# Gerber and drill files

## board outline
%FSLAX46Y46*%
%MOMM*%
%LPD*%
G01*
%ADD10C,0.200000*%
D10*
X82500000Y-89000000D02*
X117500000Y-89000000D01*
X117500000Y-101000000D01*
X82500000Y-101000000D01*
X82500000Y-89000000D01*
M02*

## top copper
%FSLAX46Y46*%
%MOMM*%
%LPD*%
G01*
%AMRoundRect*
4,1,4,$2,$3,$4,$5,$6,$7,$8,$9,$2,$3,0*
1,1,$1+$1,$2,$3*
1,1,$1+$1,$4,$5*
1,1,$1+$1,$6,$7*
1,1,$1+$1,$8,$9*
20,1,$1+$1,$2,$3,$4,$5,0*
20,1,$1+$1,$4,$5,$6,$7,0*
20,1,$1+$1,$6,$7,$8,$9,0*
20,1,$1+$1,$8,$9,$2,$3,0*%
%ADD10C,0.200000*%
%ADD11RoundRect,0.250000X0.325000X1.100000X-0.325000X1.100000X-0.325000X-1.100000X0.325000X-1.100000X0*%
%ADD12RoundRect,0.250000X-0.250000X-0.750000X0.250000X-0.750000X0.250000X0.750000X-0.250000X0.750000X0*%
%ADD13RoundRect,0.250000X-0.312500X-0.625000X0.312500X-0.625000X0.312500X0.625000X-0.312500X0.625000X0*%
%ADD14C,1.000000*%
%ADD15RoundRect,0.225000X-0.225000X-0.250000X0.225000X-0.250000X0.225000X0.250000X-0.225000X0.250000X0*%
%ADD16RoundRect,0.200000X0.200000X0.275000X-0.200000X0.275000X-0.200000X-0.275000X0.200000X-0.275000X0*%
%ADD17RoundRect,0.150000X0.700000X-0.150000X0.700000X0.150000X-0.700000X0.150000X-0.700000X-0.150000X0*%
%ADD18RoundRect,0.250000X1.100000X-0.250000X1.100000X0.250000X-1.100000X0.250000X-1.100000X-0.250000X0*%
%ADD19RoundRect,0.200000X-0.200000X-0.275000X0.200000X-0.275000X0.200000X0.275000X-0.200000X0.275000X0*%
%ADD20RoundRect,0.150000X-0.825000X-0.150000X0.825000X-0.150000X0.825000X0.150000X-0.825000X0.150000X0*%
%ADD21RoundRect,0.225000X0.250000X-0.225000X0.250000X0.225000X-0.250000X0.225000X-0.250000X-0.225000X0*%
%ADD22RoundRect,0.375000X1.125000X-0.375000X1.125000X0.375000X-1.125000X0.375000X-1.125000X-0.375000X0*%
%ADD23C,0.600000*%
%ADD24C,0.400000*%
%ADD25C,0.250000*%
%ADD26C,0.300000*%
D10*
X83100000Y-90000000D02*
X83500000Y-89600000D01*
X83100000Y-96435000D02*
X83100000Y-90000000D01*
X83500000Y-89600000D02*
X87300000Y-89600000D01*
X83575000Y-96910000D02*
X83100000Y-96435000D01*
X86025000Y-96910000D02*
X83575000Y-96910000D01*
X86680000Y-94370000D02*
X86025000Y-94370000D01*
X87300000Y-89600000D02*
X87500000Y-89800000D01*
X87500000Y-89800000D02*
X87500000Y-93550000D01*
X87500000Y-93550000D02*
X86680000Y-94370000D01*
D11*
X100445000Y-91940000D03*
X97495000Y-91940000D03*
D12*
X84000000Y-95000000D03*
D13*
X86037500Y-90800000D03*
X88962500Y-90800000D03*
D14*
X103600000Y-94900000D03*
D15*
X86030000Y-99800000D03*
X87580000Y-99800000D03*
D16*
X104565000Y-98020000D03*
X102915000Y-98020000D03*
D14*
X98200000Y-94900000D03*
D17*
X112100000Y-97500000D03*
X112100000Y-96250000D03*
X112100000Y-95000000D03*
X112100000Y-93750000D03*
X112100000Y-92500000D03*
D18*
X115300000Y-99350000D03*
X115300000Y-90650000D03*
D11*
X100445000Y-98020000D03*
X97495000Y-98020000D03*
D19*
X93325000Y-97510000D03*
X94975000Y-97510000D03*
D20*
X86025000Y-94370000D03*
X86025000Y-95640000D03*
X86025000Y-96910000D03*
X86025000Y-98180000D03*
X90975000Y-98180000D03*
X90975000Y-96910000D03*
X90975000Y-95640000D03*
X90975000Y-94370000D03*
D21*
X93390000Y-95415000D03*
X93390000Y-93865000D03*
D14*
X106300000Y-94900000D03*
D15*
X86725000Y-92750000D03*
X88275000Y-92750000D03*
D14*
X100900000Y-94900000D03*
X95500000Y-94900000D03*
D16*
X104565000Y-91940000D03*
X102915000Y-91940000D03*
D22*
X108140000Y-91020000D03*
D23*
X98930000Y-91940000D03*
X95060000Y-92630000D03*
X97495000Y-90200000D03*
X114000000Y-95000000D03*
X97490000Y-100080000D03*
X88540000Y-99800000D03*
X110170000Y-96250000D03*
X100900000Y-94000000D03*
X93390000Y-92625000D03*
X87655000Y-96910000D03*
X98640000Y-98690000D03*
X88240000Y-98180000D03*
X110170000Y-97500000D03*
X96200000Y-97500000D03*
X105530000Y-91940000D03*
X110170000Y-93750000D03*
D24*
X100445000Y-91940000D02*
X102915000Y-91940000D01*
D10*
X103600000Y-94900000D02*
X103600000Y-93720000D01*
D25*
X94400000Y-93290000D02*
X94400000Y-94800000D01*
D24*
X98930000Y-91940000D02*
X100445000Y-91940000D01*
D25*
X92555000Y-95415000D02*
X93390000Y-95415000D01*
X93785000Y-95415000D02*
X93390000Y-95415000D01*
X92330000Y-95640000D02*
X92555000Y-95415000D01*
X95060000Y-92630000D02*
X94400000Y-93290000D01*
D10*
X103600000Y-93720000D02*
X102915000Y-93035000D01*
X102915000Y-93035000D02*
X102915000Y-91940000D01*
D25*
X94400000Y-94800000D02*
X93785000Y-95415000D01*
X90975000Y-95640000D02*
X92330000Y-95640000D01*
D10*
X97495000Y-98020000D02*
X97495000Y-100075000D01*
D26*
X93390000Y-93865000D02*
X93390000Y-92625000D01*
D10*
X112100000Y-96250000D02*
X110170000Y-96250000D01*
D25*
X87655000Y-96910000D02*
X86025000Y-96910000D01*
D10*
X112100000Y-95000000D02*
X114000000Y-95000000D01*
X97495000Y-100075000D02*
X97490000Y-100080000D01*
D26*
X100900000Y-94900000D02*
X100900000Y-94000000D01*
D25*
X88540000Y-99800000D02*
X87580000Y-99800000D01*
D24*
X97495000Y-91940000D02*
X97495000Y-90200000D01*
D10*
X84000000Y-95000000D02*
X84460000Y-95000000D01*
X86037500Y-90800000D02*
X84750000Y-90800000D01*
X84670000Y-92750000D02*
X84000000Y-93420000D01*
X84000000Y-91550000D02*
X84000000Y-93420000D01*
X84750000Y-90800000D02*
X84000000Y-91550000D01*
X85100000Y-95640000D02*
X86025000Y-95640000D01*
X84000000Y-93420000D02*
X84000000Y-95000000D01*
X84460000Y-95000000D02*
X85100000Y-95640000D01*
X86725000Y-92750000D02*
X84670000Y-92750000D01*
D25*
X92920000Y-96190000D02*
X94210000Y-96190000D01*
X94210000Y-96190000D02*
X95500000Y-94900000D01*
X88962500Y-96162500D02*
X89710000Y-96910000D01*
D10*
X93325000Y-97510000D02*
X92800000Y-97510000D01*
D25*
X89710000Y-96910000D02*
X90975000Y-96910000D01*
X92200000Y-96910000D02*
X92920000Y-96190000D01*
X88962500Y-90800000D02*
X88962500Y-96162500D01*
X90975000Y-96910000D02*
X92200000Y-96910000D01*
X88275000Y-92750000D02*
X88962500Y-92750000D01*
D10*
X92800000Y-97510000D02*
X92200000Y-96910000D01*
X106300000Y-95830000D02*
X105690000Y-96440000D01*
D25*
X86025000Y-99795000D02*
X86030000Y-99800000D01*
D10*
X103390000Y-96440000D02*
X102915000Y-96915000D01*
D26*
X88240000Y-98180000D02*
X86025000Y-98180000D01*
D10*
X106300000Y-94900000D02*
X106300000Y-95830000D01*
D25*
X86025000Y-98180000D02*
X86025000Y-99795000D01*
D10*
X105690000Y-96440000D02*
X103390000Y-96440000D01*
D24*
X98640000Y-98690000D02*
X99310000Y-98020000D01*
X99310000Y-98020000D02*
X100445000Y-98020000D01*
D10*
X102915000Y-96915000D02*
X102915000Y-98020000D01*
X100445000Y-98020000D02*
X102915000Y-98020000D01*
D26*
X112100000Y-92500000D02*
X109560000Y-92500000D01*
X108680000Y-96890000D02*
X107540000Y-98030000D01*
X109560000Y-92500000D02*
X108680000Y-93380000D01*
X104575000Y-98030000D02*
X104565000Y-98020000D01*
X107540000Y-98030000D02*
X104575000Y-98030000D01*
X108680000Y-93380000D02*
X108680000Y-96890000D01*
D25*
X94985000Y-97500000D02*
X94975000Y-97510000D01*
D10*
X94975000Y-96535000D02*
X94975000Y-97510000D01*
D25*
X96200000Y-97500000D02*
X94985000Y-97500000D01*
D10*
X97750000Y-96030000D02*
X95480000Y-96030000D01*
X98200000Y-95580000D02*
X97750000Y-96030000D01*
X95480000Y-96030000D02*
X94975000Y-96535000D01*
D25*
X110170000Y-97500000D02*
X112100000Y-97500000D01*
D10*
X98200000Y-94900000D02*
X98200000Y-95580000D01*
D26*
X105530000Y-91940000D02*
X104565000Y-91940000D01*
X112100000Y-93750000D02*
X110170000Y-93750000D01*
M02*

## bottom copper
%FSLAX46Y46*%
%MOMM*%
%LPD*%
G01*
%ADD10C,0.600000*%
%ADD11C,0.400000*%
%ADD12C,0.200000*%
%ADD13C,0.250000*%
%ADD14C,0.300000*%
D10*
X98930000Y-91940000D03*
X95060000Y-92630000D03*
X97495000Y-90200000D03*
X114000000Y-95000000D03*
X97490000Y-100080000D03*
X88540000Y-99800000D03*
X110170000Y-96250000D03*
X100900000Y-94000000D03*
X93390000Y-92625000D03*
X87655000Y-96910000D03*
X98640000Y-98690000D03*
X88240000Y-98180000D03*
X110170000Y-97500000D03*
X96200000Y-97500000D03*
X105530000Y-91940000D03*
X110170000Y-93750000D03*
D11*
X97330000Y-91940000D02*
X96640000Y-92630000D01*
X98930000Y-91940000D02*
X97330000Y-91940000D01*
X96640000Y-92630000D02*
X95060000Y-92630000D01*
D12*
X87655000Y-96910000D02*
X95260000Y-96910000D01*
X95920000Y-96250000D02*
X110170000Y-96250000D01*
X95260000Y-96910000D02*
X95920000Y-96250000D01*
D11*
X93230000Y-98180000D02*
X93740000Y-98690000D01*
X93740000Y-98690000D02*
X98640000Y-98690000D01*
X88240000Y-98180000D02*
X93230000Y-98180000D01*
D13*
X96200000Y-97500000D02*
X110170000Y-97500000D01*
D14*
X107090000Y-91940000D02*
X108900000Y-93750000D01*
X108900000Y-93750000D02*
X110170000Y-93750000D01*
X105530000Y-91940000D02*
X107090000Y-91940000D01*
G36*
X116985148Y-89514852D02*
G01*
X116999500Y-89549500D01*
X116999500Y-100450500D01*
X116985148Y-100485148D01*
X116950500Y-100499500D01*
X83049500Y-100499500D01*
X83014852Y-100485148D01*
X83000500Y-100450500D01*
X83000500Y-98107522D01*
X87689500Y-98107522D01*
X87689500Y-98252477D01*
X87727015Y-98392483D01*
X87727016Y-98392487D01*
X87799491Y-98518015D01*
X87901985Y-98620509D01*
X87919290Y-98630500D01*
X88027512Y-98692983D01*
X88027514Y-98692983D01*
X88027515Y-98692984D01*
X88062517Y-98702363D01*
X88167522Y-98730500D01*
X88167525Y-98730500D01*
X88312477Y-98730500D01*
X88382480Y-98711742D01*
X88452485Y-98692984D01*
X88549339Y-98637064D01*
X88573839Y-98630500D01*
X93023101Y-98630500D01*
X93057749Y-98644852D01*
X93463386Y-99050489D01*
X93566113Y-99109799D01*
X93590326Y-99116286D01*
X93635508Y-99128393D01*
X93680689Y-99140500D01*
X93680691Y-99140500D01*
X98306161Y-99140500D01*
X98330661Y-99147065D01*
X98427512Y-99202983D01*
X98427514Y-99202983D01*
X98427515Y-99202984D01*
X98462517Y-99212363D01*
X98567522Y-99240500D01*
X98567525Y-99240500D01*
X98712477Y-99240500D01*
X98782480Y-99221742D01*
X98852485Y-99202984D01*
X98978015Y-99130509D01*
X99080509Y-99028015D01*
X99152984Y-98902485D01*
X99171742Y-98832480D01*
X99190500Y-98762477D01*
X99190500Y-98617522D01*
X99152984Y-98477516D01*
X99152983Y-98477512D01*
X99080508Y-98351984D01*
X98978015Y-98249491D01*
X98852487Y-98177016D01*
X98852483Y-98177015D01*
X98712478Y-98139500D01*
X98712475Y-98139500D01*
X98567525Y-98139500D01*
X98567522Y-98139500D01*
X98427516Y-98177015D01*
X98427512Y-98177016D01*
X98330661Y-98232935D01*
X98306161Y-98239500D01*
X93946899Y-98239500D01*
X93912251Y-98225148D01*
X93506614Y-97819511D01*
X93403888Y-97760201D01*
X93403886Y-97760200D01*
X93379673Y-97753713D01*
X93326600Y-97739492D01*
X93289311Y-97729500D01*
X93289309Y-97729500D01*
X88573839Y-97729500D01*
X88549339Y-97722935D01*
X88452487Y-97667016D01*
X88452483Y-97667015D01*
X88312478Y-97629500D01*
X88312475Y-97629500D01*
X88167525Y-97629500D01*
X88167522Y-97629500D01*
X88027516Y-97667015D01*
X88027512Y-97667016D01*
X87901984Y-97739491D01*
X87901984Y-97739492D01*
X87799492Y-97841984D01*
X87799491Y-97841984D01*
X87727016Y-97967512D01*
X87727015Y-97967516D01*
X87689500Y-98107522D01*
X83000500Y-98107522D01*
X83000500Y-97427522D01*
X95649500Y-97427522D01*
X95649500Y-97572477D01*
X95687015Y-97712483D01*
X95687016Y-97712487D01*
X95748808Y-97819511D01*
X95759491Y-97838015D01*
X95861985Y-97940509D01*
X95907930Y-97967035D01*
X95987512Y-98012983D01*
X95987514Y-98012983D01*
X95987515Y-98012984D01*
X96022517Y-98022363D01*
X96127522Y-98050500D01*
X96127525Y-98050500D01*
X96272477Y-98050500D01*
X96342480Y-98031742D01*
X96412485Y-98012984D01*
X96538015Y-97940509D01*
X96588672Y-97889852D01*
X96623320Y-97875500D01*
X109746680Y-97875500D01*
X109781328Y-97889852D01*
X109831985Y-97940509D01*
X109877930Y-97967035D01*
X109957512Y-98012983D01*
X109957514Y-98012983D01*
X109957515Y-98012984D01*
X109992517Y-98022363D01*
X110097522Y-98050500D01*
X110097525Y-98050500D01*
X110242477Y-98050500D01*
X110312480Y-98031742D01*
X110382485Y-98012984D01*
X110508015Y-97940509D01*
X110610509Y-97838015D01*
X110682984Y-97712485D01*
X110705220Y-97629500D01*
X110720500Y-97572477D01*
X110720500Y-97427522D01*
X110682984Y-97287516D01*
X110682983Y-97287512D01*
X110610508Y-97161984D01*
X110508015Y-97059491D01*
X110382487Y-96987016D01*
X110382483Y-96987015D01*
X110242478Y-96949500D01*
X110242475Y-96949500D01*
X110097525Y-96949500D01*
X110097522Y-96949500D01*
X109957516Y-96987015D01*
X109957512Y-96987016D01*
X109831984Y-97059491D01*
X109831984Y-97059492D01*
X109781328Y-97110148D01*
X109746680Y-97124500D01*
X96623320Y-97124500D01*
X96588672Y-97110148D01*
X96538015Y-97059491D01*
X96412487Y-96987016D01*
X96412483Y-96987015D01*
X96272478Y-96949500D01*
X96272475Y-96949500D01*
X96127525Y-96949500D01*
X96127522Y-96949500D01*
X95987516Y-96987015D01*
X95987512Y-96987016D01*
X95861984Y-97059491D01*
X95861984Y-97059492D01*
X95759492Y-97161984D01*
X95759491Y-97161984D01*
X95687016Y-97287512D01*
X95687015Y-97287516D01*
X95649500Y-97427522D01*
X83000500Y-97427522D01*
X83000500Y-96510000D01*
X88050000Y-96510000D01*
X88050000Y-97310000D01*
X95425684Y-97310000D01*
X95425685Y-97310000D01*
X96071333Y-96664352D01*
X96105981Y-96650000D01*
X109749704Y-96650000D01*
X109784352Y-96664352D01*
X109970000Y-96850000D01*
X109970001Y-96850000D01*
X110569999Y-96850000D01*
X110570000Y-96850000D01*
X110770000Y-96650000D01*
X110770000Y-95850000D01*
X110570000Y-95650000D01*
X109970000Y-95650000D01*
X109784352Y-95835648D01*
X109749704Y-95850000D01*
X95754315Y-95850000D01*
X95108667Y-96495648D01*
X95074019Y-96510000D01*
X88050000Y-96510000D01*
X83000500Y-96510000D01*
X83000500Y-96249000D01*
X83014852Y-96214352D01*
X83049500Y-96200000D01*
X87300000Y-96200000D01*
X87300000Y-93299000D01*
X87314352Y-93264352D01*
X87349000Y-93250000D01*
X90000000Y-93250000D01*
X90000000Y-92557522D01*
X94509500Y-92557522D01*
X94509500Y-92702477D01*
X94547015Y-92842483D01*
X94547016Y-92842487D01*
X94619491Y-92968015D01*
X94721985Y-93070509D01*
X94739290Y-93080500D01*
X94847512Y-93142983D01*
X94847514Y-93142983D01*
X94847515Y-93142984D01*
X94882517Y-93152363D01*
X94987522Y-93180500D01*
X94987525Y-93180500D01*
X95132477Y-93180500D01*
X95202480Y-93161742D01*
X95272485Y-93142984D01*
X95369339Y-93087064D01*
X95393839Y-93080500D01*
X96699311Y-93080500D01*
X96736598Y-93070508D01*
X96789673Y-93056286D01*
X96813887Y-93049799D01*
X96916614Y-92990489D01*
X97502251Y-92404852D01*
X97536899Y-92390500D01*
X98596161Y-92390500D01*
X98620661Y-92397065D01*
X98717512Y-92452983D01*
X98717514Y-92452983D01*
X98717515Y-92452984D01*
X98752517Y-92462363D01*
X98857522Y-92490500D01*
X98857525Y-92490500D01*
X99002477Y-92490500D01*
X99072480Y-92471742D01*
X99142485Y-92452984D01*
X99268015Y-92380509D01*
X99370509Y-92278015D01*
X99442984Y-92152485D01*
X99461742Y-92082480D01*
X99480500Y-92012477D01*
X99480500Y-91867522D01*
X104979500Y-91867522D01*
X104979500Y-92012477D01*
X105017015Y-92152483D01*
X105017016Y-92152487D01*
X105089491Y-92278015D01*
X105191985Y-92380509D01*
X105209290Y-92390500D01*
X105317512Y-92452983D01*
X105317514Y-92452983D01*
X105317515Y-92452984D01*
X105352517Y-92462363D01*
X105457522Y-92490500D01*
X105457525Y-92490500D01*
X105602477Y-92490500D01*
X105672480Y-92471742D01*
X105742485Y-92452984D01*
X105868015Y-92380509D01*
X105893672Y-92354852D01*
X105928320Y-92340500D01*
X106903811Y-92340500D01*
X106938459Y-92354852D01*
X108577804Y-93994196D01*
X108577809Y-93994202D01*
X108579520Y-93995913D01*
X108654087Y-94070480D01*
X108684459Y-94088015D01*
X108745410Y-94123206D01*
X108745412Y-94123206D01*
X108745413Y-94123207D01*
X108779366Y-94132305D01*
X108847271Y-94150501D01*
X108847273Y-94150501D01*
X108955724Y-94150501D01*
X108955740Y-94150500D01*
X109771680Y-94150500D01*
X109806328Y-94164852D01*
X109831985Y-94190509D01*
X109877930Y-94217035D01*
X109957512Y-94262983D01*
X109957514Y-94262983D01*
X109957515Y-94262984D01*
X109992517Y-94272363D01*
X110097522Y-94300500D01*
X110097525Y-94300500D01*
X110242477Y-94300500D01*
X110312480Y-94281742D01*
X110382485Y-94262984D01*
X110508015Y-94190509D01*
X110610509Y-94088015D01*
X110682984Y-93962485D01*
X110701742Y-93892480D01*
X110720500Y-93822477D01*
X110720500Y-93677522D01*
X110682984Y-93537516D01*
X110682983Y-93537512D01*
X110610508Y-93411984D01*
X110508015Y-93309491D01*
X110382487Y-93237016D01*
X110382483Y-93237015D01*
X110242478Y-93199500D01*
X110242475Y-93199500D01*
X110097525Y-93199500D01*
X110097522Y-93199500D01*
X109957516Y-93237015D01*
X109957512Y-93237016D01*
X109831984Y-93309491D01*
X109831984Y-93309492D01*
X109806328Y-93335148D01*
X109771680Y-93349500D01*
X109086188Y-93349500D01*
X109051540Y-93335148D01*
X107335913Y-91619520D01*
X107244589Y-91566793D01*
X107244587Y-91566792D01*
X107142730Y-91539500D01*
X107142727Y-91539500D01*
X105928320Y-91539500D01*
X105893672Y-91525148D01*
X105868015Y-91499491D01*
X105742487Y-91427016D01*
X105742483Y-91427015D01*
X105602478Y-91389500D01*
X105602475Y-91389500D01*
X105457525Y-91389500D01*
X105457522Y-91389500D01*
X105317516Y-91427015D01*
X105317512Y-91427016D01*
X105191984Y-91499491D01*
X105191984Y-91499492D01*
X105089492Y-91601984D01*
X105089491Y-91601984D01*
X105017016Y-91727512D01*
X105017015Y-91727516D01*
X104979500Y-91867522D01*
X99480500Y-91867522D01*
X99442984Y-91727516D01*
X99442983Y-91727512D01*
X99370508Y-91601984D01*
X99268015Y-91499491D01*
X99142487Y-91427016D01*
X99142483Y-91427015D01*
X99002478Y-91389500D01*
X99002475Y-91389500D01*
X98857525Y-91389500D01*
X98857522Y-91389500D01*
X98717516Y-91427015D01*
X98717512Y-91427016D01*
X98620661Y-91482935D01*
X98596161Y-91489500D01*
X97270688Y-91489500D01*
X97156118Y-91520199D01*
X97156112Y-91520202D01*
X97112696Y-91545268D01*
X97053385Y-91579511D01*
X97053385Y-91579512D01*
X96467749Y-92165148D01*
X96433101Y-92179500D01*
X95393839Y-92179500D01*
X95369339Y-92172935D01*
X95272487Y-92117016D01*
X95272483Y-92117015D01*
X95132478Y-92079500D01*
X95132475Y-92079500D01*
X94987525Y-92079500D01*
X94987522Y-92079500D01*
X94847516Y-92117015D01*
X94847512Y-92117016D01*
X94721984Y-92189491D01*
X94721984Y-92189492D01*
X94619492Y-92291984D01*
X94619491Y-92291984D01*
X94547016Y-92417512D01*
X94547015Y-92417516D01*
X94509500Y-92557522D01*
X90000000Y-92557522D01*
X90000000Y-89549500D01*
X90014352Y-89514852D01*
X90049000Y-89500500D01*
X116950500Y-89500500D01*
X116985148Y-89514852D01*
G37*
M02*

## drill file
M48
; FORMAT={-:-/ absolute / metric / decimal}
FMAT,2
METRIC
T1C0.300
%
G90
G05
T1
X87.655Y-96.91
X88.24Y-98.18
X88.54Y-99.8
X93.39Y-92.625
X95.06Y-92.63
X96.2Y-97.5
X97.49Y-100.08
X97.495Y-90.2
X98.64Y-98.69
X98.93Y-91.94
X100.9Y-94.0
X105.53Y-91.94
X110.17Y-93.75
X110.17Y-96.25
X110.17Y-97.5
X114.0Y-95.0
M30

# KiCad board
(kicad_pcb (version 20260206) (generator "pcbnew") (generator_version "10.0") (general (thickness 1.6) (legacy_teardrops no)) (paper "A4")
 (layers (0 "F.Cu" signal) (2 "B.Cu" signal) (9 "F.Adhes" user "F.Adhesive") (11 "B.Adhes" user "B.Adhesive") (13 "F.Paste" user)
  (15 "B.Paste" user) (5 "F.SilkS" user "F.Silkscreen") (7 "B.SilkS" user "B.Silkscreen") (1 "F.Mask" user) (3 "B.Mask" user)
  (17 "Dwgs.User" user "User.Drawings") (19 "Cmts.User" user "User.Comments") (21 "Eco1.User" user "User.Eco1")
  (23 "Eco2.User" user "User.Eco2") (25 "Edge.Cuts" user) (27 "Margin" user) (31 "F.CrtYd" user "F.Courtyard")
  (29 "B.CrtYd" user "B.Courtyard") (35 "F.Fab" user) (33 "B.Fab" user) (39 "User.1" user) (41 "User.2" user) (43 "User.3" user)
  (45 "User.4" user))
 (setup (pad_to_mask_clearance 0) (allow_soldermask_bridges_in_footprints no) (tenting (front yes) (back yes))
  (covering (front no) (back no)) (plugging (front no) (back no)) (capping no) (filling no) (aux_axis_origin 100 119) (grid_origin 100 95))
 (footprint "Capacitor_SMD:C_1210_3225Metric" (layer "F.Cu") (at 98.97 91.94 180)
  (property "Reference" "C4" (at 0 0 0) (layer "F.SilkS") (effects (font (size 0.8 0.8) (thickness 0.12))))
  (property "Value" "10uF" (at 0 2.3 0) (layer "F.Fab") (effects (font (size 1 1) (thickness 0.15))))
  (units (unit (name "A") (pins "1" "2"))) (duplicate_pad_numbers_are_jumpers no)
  (pad "1" smd roundrect (at -1.475 0 180) (size 1.15 2.7) (layers "F.Cu" "F.Mask" "F.Paste") (roundrect_rratio 0.217391) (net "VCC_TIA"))
  (pad "2" smd roundrect (at 1.475 0 180) (size 1.15 2.7) (layers "F.Cu" "F.Mask" "F.Paste") (roundrect_rratio 0.217391) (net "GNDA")))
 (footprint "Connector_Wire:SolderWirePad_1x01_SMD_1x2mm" (layer "F.Cu") (at 84 95)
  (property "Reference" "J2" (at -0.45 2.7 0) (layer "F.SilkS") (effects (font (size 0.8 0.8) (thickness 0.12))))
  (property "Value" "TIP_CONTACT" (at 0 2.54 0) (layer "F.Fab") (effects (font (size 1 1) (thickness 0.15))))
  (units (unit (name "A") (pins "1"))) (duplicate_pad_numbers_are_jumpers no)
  (pad "1" smd roundrect (at 0 0) (size 1 2) (layers "F.Cu" "F.Mask") (roundrect_rratio 0.25) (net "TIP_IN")))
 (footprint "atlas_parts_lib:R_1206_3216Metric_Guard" (layer "F.Cu") (at 87.5 90.8)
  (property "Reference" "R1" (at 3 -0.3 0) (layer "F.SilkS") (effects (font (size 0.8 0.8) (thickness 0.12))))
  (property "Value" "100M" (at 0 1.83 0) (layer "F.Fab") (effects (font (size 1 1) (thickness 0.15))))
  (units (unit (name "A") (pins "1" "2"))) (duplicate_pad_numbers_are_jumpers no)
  (pad "1" smd roundrect (at -1.4625 0) (size 1.125 1.75) (layers "F.Cu" "F.Mask" "F.Paste") (roundrect_rratio 0.222222) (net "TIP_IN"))
  (pad "2" smd roundrect (at 1.4625 0) (size 1.125 1.75) (layers "F.Cu" "F.Mask" "F.Paste") (roundrect_rratio 0.222222) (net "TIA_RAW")))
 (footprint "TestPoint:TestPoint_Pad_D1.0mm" (layer "F.Cu") (at 103.6 94.9)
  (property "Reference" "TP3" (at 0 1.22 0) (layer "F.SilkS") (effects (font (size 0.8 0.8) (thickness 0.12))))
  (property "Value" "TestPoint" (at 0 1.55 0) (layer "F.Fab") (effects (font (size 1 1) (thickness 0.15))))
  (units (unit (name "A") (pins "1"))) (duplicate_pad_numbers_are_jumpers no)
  (pad "1" smd circle (at 0 0) (size 1 1) (layers "F.Cu" "F.Mask") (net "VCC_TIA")))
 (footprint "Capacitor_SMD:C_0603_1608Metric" (layer "F.Cu") (at 86.805 99.8)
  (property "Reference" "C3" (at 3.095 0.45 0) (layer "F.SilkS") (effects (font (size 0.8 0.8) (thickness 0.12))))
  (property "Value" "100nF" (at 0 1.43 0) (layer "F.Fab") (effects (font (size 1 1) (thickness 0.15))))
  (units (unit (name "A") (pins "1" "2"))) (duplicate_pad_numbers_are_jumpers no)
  (pad "1" smd roundrect (at -0.775 0) (size 0.9 0.95) (layers "F.Cu" "F.Mask" "F.Paste") (roundrect_rratio 0.25) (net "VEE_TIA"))
  (pad "2" smd roundrect (at 0.775 0) (size 0.9 0.95) (layers "F.Cu" "F.Mask" "F.Paste") (roundrect_rratio 0.25) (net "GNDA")))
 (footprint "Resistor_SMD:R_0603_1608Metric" (layer "F.Cu") (at 103.74 98.02 180)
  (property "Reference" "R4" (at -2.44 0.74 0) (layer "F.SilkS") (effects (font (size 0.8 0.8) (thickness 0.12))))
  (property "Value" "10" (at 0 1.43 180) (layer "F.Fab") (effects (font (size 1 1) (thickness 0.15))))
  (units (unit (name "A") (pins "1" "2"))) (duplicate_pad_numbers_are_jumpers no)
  (pad "1" smd roundrect (at -0.825 0 180) (size 0.8 0.95) (layers "F.Cu" "F.Mask" "F.Paste") (roundrect_rratio 0.25) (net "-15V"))
  (pad "2" smd roundrect (at 0.825 0 180) (size 0.8 0.95) (layers "F.Cu" "F.Mask" "F.Paste") (roundrect_rratio 0.25) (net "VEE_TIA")))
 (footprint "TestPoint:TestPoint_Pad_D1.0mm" (layer "F.Cu") (at 98.2 94.9)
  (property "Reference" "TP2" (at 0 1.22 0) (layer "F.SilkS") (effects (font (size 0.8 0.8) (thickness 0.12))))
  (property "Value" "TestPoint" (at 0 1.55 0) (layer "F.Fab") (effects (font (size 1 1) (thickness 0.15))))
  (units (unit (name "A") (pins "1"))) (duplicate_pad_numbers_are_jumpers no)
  (pad "1" smd circle (at 0 0) (size 1 1) (layers "F.Cu" "F.Mask") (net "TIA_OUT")))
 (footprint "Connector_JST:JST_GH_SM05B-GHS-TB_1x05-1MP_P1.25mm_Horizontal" (layer "F.Cu") (at 113.95 95 90)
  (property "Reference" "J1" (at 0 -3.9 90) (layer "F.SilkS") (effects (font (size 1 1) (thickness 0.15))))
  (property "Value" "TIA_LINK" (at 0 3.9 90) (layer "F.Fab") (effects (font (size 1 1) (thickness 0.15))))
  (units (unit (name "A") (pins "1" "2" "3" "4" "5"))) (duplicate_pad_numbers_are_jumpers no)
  (pad "1" smd roundrect (at -2.5 -1.85 90) (size 0.6 1.7) (layers "F.Cu" "F.Mask" "F.Paste") (roundrect_rratio 0.25) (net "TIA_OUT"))
  (pad "2" smd roundrect (at -1.25 -1.85 90) (size 0.6 1.7) (layers "F.Cu" "F.Mask" "F.Paste") (roundrect_rratio 0.25) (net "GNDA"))
  (pad "3" smd roundrect (at 0 -1.85 90) (size 0.6 1.7) (layers "F.Cu" "F.Mask" "F.Paste") (roundrect_rratio 0.25) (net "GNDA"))
  (pad "4" smd roundrect (at 1.25 -1.85 90) (size 0.6 1.7) (layers "F.Cu" "F.Mask" "F.Paste") (roundrect_rratio 0.25) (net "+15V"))
  (pad "5" smd roundrect (at 2.5 -1.85 90) (size 0.6 1.7) (layers "F.Cu" "F.Mask" "F.Paste") (roundrect_rratio 0.25) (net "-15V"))
  (pad "MP" smd roundrect (at -4.35 1.35 90) (size 1 2.7) (layers "F.Cu" "F.Mask" "F.Paste") (roundrect_rratio 0.25))
  (pad "MP" smd roundrect (at 4.35 1.35 90) (size 1 2.7) (layers "F.Cu" "F.Mask" "F.Paste") (roundrect_rratio 0.25)))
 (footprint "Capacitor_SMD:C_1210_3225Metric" (layer "F.Cu") (at 98.97 98.02 180)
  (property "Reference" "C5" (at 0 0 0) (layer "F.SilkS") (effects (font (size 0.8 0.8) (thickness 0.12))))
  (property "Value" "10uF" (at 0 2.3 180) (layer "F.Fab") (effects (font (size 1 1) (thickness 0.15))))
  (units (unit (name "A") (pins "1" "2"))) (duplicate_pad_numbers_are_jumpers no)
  (pad "1" smd roundrect (at -1.475 0 180) (size 1.15 2.7) (layers "F.Cu" "F.Mask" "F.Paste") (roundrect_rratio 0.217391) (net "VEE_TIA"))
  (pad "2" smd roundrect (at 1.475 0 180) (size 1.15 2.7) (layers "F.Cu" "F.Mask" "F.Paste") (roundrect_rratio 0.217391) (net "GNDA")))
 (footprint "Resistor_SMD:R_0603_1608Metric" (layer "F.Cu") (at 94.15 97.51)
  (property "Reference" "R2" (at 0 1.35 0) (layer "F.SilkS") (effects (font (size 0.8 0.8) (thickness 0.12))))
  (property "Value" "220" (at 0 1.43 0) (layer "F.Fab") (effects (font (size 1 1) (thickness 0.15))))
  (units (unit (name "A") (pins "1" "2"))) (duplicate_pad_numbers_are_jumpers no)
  (pad "1" smd roundrect (at -0.825 0) (size 0.8 0.95) (layers "F.Cu" "F.Mask" "F.Paste") (roundrect_rratio 0.25) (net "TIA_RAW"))
  (pad "2" smd roundrect (at 0.825 0) (size 0.8 0.95) (layers "F.Cu" "F.Mask" "F.Paste") (roundrect_rratio 0.25) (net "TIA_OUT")))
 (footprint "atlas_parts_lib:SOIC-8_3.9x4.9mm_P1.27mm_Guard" (layer "F.Cu") (at 88.5 96.275)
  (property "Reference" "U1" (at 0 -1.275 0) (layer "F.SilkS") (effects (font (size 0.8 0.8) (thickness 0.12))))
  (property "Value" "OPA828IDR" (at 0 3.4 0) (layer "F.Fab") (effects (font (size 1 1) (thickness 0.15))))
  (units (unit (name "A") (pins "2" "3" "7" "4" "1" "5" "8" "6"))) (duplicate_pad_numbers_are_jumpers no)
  (pad "1" smd roundrect (at -2.475 -1.905) (size 1.95 0.6) (layers "F.Cu" "F.Mask" "F.Paste") (roundrect_rratio 0.25) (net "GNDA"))
  (pad "2" smd roundrect (at -2.475 -0.635) (size 1.95 0.6) (layers "F.Cu" "F.Mask" "F.Paste") (roundrect_rratio 0.25) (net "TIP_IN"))
  (pad "3" smd roundrect (at -2.475 0.635) (size 1.95 0.6) (layers "F.Cu" "F.Mask" "F.Paste") (roundrect_rratio 0.25) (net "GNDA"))
  (pad "4" smd roundrect (at -2.475 1.905) (size 1.95 0.6) (layers "F.Cu" "F.Mask" "F.Paste") (roundrect_rratio 0.25) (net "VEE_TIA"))
  (pad "5" smd roundrect (at 2.475 1.905) (size 1.95 0.6) (layers "F.Cu" "F.Mask" "F.Paste") (roundrect_rratio 0.25)
   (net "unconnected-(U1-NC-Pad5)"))
  (pad "6" smd roundrect (at 2.475 0.635) (size 1.95 0.6) (layers "F.Cu" "F.Mask" "F.Paste") (roundrect_rratio 0.25) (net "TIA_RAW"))
  (pad "7" smd roundrect (at 2.475 -0.635) (size 1.95 0.6) (layers "F.Cu" "F.Mask" "F.Paste") (roundrect_rratio 0.25) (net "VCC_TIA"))
  (pad "8" smd roundrect (at 2.475 -1.905) (size 1.95 0.6) (layers "F.Cu" "F.Mask" "F.Paste") (roundrect_rratio 0.25)
   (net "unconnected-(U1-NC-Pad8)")))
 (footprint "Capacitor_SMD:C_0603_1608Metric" (layer "F.Cu") (at 93.39 94.64 90)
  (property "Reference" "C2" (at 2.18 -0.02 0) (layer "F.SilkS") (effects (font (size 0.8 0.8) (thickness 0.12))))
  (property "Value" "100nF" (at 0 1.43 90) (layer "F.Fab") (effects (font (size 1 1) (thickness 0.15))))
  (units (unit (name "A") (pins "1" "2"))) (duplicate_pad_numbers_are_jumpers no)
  (pad "1" smd roundrect (at -0.775 0 90) (size 0.9 0.95) (layers "F.Cu" "F.Mask" "F.Paste") (roundrect_rratio 0.25) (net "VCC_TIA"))
  (pad "2" smd roundrect (at 0.775 0 90) (size 0.9 0.95) (layers "F.Cu" "F.Mask" "F.Paste") (roundrect_rratio 0.25) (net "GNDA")))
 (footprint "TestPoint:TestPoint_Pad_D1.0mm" (layer "F.Cu") (at 106.3 94.9)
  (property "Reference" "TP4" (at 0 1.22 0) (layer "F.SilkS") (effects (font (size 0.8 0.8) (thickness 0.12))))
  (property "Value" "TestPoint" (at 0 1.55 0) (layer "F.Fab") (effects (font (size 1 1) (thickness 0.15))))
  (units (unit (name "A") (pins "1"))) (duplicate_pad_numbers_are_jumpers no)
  (pad "1" smd circle (at 0 0) (size 1 1) (layers "F.Cu" "F.Mask") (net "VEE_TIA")))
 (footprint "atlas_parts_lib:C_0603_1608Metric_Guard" (layer "F.Cu") (at 87.5 92.75)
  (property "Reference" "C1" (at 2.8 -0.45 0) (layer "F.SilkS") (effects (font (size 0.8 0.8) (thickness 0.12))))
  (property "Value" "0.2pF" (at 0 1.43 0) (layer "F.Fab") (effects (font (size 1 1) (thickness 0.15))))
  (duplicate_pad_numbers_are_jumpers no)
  (pad "1" smd roundrect (at -0.775 0) (size 0.9 0.95) (layers "F.Cu" "F.Mask" "F.Paste") (roundrect_rratio 0.25) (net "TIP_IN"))
  (pad "2" smd roundrect (at 0.775 0) (size 0.9 0.95) (layers "F.Cu" "F.Mask" "F.Paste") (roundrect_rratio 0.25) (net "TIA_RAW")))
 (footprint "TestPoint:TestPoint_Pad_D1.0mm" (layer "F.Cu") (at 100.9 94.9)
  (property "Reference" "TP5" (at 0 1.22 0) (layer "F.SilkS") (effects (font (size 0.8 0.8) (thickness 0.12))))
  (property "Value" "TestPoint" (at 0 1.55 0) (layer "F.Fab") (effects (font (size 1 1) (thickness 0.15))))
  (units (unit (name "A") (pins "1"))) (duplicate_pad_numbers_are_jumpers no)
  (pad "1" smd circle (at 0 0) (size 1 1) (layers "F.Cu" "F.Mask") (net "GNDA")))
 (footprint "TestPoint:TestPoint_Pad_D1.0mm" (layer "F.Cu") (at 95.5 94.9)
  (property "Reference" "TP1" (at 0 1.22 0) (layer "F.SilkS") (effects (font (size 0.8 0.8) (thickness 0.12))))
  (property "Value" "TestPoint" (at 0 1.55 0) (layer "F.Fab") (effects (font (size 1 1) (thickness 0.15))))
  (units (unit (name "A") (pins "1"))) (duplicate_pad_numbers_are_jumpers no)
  (pad "1" smd circle (at 0 0) (size 1 1) (layers "F.Cu" "F.Mask") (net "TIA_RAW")))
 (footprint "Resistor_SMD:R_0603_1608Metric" (layer "F.Cu") (at 103.74 91.94 180)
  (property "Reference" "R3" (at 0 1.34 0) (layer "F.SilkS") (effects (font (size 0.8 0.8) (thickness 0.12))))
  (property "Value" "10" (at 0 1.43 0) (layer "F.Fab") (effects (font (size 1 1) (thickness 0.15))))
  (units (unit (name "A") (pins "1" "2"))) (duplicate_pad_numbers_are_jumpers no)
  (pad "1" smd roundrect (at -0.825 0 180) (size 0.8 0.95) (layers "F.Cu" "F.Mask" "F.Paste") (roundrect_rratio 0.25) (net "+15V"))
  (pad "2" smd roundrect (at 0.825 0 180) (size 0.8 0.95) (layers "F.Cu" "F.Mask" "F.Paste") (roundrect_rratio 0.25) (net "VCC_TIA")))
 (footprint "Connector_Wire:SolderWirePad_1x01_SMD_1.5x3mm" (layer "F.Cu") (at 108.14 91.02 90)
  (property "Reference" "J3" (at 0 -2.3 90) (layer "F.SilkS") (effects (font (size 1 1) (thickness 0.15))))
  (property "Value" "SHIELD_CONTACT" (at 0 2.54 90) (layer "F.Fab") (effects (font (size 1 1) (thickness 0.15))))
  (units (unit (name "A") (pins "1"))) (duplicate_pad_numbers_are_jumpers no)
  (pad "1" smd roundrect (at 0 0 90) (size 1.5 3) (layers "F.Cu" "F.Mask") (roundrect_rratio 0.25) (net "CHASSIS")))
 (gr_line (start 83.1 90) (end 83.5 89.6) (stroke (width 0.2) (type default)) (layer "F.Cu") (net "GNDA"))
 (gr_line (start 83.1 96.435) (end 83.1 90) (stroke (width 0.2) (type default)) (layer "F.Cu") (net "GNDA"))
 (gr_line (start 83.5 89.6) (end 87.3 89.6) (stroke (width 0.2) (type default)) (layer "F.Cu") (net "GNDA"))
 (gr_line (start 83.575 96.91) (end 83.1 96.435) (stroke (width 0.2) (type default)) (layer "F.Cu") (net "GNDA"))
 (gr_line (start 86.025 96.91) (end 83.575 96.91) (stroke (width 0.2) (type default)) (layer "F.Cu") (net "GNDA"))
 (gr_line (start 86.68 94.37) (end 86.025 94.37) (stroke (width 0.2) (type default)) (layer "F.Cu") (net "GNDA"))
 (gr_line (start 87.3 89.6) (end 87.5 89.8) (stroke (width 0.2) (type default)) (layer "F.Cu") (net "GNDA"))
 (gr_line (start 87.5 89.8) (end 87.5 93.55) (stroke (width 0.2) (type default)) (layer "F.Cu") (net "GNDA"))
 (gr_line (start 87.5 93.55) (end 86.68 94.37) (stroke (width 0.2) (type default)) (layer "F.Cu") (net "GNDA"))
 (gr_rect (start 82.5 89) (end 117.5 101) (stroke (width 0.2) (type solid)) (fill no) (layer "Edge.Cuts"))
 (segment (start 100.445 91.94) (end 102.915 91.94) (width 0.4) (layer "F.Cu") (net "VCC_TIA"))
 (segment (start 103.6 94.9) (end 103.6 93.72) (width 0.2) (layer "F.Cu") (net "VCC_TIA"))
 (segment (start 94.4 93.29) (end 94.4 94.8) (width 0.25) (layer "F.Cu") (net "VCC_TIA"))
 (segment (start 98.93 91.94) (end 100.445 91.94) (width 0.4) (layer "F.Cu") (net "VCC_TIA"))
 (segment (start 92.555 95.415) (end 93.39 95.415) (width 0.25) (layer "F.Cu") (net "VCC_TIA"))
 (segment (start 93.785 95.415) (end 93.39 95.415) (width 0.25) (layer "F.Cu") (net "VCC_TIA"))
 (segment (start 92.33 95.64) (end 92.555 95.415) (width 0.25) (layer "F.Cu") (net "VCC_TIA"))
 (segment (start 95.06 92.63) (end 94.4 93.29) (width 0.25) (layer "F.Cu") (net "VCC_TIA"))
 (segment (start 103.6 93.72) (end 102.915 93.035) (width 0.2) (layer "F.Cu") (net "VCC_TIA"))
 (segment (start 102.915 93.035) (end 102.915 91.94) (width 0.2) (layer "F.Cu") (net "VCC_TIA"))
 (segment (start 94.4 94.8) (end 93.785 95.415) (width 0.25) (layer "F.Cu") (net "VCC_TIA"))
 (segment (start 90.975 95.64) (end 92.33 95.64) (width 0.25) (layer "F.Cu") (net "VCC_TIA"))
 (via (at 98.93 91.94) (size 0.6) (drill 0.3) (layers "F.Cu" "B.Cu") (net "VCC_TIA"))
 (via (at 95.06 92.63) (size 0.6) (drill 0.3) (layers "F.Cu" "B.Cu") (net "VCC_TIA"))
 (segment (start 97.33 91.94) (end 96.64 92.63) (width 0.4) (layer "B.Cu") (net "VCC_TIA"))
 (segment (start 98.93 91.94) (end 97.33 91.94) (width 0.4) (layer "B.Cu") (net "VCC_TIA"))
 (segment (start 96.64 92.63) (end 95.06 92.63) (width 0.4) (layer "B.Cu") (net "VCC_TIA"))
 (segment (start 97.495 98.02) (end 97.495 100.075) (width 0.2) (layer "F.Cu") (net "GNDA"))
 (segment (start 93.39 93.865) (end 93.39 92.625) (width 0.3) (layer "F.Cu") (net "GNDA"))
 (segment (start 112.1 96.25) (end 110.17 96.25) (width 0.2) (layer "F.Cu") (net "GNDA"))
 (segment (start 87.655 96.91) (end 86.025 96.91) (width 0.25) (layer "F.Cu") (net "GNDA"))
 (segment (start 112.1 95) (end 114 95) (width 0.2) (layer "F.Cu") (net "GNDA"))
 (segment (start 97.495 100.075) (end 97.49 100.08) (width 0.2) (layer "F.Cu") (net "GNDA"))
 (segment (start 100.9 94.9) (end 100.9 94) (width 0.3) (layer "F.Cu") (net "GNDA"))
 (segment (start 88.54 99.8) (end 87.58 99.8) (width 0.25) (layer "F.Cu") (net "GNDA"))
 (segment (start 97.495 91.94) (end 97.495 90.2) (width 0.4) (layer "F.Cu") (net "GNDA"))
 (via (at 97.495 90.2) (size 0.6) (drill 0.3) (layers "F.Cu" "B.Cu") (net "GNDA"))
 (via (at 114 95) (size 0.6) (drill 0.3) (layers "F.Cu" "B.Cu") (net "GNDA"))
 (via (at 97.49 100.08) (size 0.6) (drill 0.3) (layers "F.Cu" "B.Cu") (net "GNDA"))
 (via (at 88.54 99.8) (size 0.6) (drill 0.3) (layers "F.Cu" "B.Cu") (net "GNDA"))
 (via (at 110.17 96.25) (size 0.6) (drill 0.3) (layers "F.Cu" "B.Cu") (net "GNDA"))
 (via (at 100.9 94) (size 0.6) (drill 0.3) (layers "F.Cu" "B.Cu") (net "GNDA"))
 (via (at 93.39 92.625) (size 0.6) (drill 0.3) (layers "F.Cu" "B.Cu") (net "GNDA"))
 (via (at 87.655 96.91) (size 0.6) (drill 0.3) (layers "F.Cu" "B.Cu") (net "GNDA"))
 (segment (start 87.655 96.91) (end 95.26 96.91) (width 0.2) (layer "B.Cu") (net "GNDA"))
 (segment (start 95.92 96.25) (end 110.17 96.25) (width 0.2) (layer "B.Cu") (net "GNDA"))
 (segment (start 95.26 96.91) (end 95.92 96.25) (width 0.2) (layer "B.Cu") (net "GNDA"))
 (segment (start 84 95) (end 84.46 95) (width 0.2) (layer "F.Cu") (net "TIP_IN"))
 (segment (start 86.0375 90.8) (end 84.75 90.8) (width 0.2) (layer "F.Cu") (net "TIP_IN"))
 (segment (start 84.67 92.75) (end 84 93.42) (width 0.2) (layer "F.Cu") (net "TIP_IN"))
 (segment (start 84 91.55) (end 84 93.42) (width 0.2) (layer "F.Cu") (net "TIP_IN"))
 (segment (start 84.75 90.8) (end 84 91.55) (width 0.2) (layer "F.Cu") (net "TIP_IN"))
 (segment (start 85.1 95.64) (end 86.025 95.64) (width 0.2) (layer "F.Cu") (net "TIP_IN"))
 (segment (start 84 93.42) (end 84 95) (width 0.2) (layer "F.Cu") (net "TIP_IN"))
 (segment (start 84.46 95) (end 85.1 95.64) (width 0.2) (layer "F.Cu") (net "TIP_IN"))
 (segment (start 86.725 92.75) (end 84.67 92.75) (width 0.2) (layer "F.Cu") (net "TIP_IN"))
 (segment (start 92.92 96.19) (end 94.21 96.19) (width 0.25) (layer "F.Cu") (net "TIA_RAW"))
 (segment (start 94.21 96.19) (end 95.5 94.9) (width 0.25) (layer "F.Cu") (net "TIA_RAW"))
 (segment (start 88.9625 96.1625) (end 89.71 96.91) (width 0.25) (layer "F.Cu") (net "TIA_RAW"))
 (segment (start 93.325 97.51) (end 92.8 97.51) (width 0.2) (layer "F.Cu") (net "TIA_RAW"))
 (segment (start 89.71 96.91) (end 90.975 96.91) (width 0.25) (layer "F.Cu") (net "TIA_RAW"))
 (segment (start 92.2 96.91) (end 92.92 96.19) (width 0.25) (layer "F.Cu") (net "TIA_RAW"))
 (segment (start 88.9625 90.8) (end 88.9625 96.1625) (width 0.25) (layer "F.Cu") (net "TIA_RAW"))
 (segment (start 90.975 96.91) (end 92.2 96.91) (width 0.25) (layer "F.Cu") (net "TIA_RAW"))
 (segment (start 88.275 92.75) (end 88.9625 92.75) (width 0.25) (layer "F.Cu") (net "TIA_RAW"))
 (segment (start 92.8 97.51) (end 92.2 96.91) (width 0.2) (layer "F.Cu") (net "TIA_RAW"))
 (segment (start 106.3 95.83) (end 105.69 96.44) (width 0.2) (layer "F.Cu") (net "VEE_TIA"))
 (segment (start 86.025 99.795) (end 86.03 99.8) (width 0.25) (layer "F.Cu") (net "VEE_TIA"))
 (segment (start 103.39 96.44) (end 102.915 96.915) (width 0.2) (layer "F.Cu") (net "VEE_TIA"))
 (segment (start 88.24 98.18) (end 86.025 98.18) (width 0.3) (layer "F.Cu") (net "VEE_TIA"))
 (segment (start 106.3 94.9) (end 106.3 95.83) (width 0.2) (layer "F.Cu") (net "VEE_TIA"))
 (segment (start 86.025 98.18) (end 86.025 99.795) (width 0.25) (layer "F.Cu") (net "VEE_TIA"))
 (segment (start 105.69 96.44) (end 103.39 96.44) (width 0.2) (layer "F.Cu") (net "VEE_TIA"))
 (segment (start 98.64 98.69) (end 99.31 98.02) (width 0.4) (layer "F.Cu") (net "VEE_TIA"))
 (segment (start 99.31 98.02) (end 100.445 98.02) (width 0.4) (layer "F.Cu") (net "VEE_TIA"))
 (segment (start 102.915 96.915) (end 102.915 98.02) (width 0.2) (layer "F.Cu") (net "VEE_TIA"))
 (segment (start 100.445 98.02) (end 102.915 98.02) (width 0.2) (layer "F.Cu") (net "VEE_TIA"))
 (via (at 98.64 98.69) (size 0.6) (drill 0.3) (layers "F.Cu" "B.Cu") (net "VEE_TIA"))
 (via (at 88.24 98.18) (size 0.6) (drill 0.3) (layers "F.Cu" "B.Cu") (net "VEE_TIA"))
 (segment (start 93.23 98.18) (end 93.74 98.69) (width 0.4) (layer "B.Cu") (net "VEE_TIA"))
 (segment (start 93.74 98.69) (end 98.64 98.69) (width 0.4) (layer "B.Cu") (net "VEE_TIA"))
 (segment (start 88.24 98.18) (end 93.23 98.18) (width 0.4) (layer "B.Cu") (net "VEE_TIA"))
 (segment (start 112.1 92.5) (end 109.56 92.5) (width 0.3) (layer "F.Cu") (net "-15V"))
 (segment (start 108.68 96.89) (end 107.54 98.03) (width 0.3) (layer "F.Cu") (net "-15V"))
 (segment (start 109.56 92.5) (end 108.68 93.38) (width 0.3) (layer "F.Cu") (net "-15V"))
 (segment (start 104.575 98.03) (end 104.565 98.02) (width 0.3) (layer "F.Cu") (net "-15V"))
 (segment (start 107.54 98.03) (end 104.575 98.03) (width 0.3) (layer "F.Cu") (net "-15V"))
 (segment (start 108.68 93.38) (end 108.68 96.89) (width 0.3) (layer "F.Cu") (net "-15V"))
 (segment (start 94.985 97.5) (end 94.975 97.51) (width 0.25) (layer "F.Cu") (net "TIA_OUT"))
 (segment (start 94.975 96.535) (end 94.975 97.51) (width 0.2) (layer "F.Cu") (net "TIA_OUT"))
 (segment (start 96.2 97.5) (end 94.985 97.5) (width 0.25) (layer "F.Cu") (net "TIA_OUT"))
 (segment (start 97.75 96.03) (end 95.48 96.03) (width 0.2) (layer "F.Cu") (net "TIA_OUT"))
 (segment (start 98.2 95.58) (end 97.75 96.03) (width 0.2) (layer "F.Cu") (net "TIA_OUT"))
 (segment (start 95.48 96.03) (end 94.975 96.535) (width 0.2) (layer "F.Cu") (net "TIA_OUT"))
 (segment (start 110.17 97.5) (end 112.1 97.5) (width 0.25) (layer "F.Cu") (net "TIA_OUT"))
 (segment (start 98.2 94.9) (end 98.2 95.58) (width 0.2) (layer "F.Cu") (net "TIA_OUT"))
 (via (at 110.17 97.5) (size 0.6) (drill 0.3) (layers "F.Cu" "B.Cu") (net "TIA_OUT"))
 (via (at 96.2 97.5) (size 0.6) (drill 0.3) (layers "F.Cu" "B.Cu") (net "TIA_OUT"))
 (segment (start 96.2 97.5) (end 110.17 97.5) (width 0.25) (layer "B.Cu") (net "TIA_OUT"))
 (segment (start 105.53 91.94) (end 104.565 91.94) (width 0.3) (layer "F.Cu") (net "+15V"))
 (segment (start 112.1 93.75) (end 110.17 93.75) (width 0.3) (layer "F.Cu") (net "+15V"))
 (via (at 105.53 91.94) (size 0.6) (drill 0.3) (layers "F.Cu" "B.Cu") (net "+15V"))
 (via (at 110.17 93.75) (size 0.6) (drill 0.3) (layers "F.Cu" "B.Cu") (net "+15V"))
 (segment (start 107.09 91.94) (end 108.9 93.75) (width 0.3) (layer "B.Cu") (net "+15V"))
 (segment (start 108.9 93.75) (end 110.17 93.75) (width 0.3) (layer "B.Cu") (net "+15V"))
 (segment (start 105.53 91.94) (end 107.09 91.94) (width 0.3) (layer "B.Cu") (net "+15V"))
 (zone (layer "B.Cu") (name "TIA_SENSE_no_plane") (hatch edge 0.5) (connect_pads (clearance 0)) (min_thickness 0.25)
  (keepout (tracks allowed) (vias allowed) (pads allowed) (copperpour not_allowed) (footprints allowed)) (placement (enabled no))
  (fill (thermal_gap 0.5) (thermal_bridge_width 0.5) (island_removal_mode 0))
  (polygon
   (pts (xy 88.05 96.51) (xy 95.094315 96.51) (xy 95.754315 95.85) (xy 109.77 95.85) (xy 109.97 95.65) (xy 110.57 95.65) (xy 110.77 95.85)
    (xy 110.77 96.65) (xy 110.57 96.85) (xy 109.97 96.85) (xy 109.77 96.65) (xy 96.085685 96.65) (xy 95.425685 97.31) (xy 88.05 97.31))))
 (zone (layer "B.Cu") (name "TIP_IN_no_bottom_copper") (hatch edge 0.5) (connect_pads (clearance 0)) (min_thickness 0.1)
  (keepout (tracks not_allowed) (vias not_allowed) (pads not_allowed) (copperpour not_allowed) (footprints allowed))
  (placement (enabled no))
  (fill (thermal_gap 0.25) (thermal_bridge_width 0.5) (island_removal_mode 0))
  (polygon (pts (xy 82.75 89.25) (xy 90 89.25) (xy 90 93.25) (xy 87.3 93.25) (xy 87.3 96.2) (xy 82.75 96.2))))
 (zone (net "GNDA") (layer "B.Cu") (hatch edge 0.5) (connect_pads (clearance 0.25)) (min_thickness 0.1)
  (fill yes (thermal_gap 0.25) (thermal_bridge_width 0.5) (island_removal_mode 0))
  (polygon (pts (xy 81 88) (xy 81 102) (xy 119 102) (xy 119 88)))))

